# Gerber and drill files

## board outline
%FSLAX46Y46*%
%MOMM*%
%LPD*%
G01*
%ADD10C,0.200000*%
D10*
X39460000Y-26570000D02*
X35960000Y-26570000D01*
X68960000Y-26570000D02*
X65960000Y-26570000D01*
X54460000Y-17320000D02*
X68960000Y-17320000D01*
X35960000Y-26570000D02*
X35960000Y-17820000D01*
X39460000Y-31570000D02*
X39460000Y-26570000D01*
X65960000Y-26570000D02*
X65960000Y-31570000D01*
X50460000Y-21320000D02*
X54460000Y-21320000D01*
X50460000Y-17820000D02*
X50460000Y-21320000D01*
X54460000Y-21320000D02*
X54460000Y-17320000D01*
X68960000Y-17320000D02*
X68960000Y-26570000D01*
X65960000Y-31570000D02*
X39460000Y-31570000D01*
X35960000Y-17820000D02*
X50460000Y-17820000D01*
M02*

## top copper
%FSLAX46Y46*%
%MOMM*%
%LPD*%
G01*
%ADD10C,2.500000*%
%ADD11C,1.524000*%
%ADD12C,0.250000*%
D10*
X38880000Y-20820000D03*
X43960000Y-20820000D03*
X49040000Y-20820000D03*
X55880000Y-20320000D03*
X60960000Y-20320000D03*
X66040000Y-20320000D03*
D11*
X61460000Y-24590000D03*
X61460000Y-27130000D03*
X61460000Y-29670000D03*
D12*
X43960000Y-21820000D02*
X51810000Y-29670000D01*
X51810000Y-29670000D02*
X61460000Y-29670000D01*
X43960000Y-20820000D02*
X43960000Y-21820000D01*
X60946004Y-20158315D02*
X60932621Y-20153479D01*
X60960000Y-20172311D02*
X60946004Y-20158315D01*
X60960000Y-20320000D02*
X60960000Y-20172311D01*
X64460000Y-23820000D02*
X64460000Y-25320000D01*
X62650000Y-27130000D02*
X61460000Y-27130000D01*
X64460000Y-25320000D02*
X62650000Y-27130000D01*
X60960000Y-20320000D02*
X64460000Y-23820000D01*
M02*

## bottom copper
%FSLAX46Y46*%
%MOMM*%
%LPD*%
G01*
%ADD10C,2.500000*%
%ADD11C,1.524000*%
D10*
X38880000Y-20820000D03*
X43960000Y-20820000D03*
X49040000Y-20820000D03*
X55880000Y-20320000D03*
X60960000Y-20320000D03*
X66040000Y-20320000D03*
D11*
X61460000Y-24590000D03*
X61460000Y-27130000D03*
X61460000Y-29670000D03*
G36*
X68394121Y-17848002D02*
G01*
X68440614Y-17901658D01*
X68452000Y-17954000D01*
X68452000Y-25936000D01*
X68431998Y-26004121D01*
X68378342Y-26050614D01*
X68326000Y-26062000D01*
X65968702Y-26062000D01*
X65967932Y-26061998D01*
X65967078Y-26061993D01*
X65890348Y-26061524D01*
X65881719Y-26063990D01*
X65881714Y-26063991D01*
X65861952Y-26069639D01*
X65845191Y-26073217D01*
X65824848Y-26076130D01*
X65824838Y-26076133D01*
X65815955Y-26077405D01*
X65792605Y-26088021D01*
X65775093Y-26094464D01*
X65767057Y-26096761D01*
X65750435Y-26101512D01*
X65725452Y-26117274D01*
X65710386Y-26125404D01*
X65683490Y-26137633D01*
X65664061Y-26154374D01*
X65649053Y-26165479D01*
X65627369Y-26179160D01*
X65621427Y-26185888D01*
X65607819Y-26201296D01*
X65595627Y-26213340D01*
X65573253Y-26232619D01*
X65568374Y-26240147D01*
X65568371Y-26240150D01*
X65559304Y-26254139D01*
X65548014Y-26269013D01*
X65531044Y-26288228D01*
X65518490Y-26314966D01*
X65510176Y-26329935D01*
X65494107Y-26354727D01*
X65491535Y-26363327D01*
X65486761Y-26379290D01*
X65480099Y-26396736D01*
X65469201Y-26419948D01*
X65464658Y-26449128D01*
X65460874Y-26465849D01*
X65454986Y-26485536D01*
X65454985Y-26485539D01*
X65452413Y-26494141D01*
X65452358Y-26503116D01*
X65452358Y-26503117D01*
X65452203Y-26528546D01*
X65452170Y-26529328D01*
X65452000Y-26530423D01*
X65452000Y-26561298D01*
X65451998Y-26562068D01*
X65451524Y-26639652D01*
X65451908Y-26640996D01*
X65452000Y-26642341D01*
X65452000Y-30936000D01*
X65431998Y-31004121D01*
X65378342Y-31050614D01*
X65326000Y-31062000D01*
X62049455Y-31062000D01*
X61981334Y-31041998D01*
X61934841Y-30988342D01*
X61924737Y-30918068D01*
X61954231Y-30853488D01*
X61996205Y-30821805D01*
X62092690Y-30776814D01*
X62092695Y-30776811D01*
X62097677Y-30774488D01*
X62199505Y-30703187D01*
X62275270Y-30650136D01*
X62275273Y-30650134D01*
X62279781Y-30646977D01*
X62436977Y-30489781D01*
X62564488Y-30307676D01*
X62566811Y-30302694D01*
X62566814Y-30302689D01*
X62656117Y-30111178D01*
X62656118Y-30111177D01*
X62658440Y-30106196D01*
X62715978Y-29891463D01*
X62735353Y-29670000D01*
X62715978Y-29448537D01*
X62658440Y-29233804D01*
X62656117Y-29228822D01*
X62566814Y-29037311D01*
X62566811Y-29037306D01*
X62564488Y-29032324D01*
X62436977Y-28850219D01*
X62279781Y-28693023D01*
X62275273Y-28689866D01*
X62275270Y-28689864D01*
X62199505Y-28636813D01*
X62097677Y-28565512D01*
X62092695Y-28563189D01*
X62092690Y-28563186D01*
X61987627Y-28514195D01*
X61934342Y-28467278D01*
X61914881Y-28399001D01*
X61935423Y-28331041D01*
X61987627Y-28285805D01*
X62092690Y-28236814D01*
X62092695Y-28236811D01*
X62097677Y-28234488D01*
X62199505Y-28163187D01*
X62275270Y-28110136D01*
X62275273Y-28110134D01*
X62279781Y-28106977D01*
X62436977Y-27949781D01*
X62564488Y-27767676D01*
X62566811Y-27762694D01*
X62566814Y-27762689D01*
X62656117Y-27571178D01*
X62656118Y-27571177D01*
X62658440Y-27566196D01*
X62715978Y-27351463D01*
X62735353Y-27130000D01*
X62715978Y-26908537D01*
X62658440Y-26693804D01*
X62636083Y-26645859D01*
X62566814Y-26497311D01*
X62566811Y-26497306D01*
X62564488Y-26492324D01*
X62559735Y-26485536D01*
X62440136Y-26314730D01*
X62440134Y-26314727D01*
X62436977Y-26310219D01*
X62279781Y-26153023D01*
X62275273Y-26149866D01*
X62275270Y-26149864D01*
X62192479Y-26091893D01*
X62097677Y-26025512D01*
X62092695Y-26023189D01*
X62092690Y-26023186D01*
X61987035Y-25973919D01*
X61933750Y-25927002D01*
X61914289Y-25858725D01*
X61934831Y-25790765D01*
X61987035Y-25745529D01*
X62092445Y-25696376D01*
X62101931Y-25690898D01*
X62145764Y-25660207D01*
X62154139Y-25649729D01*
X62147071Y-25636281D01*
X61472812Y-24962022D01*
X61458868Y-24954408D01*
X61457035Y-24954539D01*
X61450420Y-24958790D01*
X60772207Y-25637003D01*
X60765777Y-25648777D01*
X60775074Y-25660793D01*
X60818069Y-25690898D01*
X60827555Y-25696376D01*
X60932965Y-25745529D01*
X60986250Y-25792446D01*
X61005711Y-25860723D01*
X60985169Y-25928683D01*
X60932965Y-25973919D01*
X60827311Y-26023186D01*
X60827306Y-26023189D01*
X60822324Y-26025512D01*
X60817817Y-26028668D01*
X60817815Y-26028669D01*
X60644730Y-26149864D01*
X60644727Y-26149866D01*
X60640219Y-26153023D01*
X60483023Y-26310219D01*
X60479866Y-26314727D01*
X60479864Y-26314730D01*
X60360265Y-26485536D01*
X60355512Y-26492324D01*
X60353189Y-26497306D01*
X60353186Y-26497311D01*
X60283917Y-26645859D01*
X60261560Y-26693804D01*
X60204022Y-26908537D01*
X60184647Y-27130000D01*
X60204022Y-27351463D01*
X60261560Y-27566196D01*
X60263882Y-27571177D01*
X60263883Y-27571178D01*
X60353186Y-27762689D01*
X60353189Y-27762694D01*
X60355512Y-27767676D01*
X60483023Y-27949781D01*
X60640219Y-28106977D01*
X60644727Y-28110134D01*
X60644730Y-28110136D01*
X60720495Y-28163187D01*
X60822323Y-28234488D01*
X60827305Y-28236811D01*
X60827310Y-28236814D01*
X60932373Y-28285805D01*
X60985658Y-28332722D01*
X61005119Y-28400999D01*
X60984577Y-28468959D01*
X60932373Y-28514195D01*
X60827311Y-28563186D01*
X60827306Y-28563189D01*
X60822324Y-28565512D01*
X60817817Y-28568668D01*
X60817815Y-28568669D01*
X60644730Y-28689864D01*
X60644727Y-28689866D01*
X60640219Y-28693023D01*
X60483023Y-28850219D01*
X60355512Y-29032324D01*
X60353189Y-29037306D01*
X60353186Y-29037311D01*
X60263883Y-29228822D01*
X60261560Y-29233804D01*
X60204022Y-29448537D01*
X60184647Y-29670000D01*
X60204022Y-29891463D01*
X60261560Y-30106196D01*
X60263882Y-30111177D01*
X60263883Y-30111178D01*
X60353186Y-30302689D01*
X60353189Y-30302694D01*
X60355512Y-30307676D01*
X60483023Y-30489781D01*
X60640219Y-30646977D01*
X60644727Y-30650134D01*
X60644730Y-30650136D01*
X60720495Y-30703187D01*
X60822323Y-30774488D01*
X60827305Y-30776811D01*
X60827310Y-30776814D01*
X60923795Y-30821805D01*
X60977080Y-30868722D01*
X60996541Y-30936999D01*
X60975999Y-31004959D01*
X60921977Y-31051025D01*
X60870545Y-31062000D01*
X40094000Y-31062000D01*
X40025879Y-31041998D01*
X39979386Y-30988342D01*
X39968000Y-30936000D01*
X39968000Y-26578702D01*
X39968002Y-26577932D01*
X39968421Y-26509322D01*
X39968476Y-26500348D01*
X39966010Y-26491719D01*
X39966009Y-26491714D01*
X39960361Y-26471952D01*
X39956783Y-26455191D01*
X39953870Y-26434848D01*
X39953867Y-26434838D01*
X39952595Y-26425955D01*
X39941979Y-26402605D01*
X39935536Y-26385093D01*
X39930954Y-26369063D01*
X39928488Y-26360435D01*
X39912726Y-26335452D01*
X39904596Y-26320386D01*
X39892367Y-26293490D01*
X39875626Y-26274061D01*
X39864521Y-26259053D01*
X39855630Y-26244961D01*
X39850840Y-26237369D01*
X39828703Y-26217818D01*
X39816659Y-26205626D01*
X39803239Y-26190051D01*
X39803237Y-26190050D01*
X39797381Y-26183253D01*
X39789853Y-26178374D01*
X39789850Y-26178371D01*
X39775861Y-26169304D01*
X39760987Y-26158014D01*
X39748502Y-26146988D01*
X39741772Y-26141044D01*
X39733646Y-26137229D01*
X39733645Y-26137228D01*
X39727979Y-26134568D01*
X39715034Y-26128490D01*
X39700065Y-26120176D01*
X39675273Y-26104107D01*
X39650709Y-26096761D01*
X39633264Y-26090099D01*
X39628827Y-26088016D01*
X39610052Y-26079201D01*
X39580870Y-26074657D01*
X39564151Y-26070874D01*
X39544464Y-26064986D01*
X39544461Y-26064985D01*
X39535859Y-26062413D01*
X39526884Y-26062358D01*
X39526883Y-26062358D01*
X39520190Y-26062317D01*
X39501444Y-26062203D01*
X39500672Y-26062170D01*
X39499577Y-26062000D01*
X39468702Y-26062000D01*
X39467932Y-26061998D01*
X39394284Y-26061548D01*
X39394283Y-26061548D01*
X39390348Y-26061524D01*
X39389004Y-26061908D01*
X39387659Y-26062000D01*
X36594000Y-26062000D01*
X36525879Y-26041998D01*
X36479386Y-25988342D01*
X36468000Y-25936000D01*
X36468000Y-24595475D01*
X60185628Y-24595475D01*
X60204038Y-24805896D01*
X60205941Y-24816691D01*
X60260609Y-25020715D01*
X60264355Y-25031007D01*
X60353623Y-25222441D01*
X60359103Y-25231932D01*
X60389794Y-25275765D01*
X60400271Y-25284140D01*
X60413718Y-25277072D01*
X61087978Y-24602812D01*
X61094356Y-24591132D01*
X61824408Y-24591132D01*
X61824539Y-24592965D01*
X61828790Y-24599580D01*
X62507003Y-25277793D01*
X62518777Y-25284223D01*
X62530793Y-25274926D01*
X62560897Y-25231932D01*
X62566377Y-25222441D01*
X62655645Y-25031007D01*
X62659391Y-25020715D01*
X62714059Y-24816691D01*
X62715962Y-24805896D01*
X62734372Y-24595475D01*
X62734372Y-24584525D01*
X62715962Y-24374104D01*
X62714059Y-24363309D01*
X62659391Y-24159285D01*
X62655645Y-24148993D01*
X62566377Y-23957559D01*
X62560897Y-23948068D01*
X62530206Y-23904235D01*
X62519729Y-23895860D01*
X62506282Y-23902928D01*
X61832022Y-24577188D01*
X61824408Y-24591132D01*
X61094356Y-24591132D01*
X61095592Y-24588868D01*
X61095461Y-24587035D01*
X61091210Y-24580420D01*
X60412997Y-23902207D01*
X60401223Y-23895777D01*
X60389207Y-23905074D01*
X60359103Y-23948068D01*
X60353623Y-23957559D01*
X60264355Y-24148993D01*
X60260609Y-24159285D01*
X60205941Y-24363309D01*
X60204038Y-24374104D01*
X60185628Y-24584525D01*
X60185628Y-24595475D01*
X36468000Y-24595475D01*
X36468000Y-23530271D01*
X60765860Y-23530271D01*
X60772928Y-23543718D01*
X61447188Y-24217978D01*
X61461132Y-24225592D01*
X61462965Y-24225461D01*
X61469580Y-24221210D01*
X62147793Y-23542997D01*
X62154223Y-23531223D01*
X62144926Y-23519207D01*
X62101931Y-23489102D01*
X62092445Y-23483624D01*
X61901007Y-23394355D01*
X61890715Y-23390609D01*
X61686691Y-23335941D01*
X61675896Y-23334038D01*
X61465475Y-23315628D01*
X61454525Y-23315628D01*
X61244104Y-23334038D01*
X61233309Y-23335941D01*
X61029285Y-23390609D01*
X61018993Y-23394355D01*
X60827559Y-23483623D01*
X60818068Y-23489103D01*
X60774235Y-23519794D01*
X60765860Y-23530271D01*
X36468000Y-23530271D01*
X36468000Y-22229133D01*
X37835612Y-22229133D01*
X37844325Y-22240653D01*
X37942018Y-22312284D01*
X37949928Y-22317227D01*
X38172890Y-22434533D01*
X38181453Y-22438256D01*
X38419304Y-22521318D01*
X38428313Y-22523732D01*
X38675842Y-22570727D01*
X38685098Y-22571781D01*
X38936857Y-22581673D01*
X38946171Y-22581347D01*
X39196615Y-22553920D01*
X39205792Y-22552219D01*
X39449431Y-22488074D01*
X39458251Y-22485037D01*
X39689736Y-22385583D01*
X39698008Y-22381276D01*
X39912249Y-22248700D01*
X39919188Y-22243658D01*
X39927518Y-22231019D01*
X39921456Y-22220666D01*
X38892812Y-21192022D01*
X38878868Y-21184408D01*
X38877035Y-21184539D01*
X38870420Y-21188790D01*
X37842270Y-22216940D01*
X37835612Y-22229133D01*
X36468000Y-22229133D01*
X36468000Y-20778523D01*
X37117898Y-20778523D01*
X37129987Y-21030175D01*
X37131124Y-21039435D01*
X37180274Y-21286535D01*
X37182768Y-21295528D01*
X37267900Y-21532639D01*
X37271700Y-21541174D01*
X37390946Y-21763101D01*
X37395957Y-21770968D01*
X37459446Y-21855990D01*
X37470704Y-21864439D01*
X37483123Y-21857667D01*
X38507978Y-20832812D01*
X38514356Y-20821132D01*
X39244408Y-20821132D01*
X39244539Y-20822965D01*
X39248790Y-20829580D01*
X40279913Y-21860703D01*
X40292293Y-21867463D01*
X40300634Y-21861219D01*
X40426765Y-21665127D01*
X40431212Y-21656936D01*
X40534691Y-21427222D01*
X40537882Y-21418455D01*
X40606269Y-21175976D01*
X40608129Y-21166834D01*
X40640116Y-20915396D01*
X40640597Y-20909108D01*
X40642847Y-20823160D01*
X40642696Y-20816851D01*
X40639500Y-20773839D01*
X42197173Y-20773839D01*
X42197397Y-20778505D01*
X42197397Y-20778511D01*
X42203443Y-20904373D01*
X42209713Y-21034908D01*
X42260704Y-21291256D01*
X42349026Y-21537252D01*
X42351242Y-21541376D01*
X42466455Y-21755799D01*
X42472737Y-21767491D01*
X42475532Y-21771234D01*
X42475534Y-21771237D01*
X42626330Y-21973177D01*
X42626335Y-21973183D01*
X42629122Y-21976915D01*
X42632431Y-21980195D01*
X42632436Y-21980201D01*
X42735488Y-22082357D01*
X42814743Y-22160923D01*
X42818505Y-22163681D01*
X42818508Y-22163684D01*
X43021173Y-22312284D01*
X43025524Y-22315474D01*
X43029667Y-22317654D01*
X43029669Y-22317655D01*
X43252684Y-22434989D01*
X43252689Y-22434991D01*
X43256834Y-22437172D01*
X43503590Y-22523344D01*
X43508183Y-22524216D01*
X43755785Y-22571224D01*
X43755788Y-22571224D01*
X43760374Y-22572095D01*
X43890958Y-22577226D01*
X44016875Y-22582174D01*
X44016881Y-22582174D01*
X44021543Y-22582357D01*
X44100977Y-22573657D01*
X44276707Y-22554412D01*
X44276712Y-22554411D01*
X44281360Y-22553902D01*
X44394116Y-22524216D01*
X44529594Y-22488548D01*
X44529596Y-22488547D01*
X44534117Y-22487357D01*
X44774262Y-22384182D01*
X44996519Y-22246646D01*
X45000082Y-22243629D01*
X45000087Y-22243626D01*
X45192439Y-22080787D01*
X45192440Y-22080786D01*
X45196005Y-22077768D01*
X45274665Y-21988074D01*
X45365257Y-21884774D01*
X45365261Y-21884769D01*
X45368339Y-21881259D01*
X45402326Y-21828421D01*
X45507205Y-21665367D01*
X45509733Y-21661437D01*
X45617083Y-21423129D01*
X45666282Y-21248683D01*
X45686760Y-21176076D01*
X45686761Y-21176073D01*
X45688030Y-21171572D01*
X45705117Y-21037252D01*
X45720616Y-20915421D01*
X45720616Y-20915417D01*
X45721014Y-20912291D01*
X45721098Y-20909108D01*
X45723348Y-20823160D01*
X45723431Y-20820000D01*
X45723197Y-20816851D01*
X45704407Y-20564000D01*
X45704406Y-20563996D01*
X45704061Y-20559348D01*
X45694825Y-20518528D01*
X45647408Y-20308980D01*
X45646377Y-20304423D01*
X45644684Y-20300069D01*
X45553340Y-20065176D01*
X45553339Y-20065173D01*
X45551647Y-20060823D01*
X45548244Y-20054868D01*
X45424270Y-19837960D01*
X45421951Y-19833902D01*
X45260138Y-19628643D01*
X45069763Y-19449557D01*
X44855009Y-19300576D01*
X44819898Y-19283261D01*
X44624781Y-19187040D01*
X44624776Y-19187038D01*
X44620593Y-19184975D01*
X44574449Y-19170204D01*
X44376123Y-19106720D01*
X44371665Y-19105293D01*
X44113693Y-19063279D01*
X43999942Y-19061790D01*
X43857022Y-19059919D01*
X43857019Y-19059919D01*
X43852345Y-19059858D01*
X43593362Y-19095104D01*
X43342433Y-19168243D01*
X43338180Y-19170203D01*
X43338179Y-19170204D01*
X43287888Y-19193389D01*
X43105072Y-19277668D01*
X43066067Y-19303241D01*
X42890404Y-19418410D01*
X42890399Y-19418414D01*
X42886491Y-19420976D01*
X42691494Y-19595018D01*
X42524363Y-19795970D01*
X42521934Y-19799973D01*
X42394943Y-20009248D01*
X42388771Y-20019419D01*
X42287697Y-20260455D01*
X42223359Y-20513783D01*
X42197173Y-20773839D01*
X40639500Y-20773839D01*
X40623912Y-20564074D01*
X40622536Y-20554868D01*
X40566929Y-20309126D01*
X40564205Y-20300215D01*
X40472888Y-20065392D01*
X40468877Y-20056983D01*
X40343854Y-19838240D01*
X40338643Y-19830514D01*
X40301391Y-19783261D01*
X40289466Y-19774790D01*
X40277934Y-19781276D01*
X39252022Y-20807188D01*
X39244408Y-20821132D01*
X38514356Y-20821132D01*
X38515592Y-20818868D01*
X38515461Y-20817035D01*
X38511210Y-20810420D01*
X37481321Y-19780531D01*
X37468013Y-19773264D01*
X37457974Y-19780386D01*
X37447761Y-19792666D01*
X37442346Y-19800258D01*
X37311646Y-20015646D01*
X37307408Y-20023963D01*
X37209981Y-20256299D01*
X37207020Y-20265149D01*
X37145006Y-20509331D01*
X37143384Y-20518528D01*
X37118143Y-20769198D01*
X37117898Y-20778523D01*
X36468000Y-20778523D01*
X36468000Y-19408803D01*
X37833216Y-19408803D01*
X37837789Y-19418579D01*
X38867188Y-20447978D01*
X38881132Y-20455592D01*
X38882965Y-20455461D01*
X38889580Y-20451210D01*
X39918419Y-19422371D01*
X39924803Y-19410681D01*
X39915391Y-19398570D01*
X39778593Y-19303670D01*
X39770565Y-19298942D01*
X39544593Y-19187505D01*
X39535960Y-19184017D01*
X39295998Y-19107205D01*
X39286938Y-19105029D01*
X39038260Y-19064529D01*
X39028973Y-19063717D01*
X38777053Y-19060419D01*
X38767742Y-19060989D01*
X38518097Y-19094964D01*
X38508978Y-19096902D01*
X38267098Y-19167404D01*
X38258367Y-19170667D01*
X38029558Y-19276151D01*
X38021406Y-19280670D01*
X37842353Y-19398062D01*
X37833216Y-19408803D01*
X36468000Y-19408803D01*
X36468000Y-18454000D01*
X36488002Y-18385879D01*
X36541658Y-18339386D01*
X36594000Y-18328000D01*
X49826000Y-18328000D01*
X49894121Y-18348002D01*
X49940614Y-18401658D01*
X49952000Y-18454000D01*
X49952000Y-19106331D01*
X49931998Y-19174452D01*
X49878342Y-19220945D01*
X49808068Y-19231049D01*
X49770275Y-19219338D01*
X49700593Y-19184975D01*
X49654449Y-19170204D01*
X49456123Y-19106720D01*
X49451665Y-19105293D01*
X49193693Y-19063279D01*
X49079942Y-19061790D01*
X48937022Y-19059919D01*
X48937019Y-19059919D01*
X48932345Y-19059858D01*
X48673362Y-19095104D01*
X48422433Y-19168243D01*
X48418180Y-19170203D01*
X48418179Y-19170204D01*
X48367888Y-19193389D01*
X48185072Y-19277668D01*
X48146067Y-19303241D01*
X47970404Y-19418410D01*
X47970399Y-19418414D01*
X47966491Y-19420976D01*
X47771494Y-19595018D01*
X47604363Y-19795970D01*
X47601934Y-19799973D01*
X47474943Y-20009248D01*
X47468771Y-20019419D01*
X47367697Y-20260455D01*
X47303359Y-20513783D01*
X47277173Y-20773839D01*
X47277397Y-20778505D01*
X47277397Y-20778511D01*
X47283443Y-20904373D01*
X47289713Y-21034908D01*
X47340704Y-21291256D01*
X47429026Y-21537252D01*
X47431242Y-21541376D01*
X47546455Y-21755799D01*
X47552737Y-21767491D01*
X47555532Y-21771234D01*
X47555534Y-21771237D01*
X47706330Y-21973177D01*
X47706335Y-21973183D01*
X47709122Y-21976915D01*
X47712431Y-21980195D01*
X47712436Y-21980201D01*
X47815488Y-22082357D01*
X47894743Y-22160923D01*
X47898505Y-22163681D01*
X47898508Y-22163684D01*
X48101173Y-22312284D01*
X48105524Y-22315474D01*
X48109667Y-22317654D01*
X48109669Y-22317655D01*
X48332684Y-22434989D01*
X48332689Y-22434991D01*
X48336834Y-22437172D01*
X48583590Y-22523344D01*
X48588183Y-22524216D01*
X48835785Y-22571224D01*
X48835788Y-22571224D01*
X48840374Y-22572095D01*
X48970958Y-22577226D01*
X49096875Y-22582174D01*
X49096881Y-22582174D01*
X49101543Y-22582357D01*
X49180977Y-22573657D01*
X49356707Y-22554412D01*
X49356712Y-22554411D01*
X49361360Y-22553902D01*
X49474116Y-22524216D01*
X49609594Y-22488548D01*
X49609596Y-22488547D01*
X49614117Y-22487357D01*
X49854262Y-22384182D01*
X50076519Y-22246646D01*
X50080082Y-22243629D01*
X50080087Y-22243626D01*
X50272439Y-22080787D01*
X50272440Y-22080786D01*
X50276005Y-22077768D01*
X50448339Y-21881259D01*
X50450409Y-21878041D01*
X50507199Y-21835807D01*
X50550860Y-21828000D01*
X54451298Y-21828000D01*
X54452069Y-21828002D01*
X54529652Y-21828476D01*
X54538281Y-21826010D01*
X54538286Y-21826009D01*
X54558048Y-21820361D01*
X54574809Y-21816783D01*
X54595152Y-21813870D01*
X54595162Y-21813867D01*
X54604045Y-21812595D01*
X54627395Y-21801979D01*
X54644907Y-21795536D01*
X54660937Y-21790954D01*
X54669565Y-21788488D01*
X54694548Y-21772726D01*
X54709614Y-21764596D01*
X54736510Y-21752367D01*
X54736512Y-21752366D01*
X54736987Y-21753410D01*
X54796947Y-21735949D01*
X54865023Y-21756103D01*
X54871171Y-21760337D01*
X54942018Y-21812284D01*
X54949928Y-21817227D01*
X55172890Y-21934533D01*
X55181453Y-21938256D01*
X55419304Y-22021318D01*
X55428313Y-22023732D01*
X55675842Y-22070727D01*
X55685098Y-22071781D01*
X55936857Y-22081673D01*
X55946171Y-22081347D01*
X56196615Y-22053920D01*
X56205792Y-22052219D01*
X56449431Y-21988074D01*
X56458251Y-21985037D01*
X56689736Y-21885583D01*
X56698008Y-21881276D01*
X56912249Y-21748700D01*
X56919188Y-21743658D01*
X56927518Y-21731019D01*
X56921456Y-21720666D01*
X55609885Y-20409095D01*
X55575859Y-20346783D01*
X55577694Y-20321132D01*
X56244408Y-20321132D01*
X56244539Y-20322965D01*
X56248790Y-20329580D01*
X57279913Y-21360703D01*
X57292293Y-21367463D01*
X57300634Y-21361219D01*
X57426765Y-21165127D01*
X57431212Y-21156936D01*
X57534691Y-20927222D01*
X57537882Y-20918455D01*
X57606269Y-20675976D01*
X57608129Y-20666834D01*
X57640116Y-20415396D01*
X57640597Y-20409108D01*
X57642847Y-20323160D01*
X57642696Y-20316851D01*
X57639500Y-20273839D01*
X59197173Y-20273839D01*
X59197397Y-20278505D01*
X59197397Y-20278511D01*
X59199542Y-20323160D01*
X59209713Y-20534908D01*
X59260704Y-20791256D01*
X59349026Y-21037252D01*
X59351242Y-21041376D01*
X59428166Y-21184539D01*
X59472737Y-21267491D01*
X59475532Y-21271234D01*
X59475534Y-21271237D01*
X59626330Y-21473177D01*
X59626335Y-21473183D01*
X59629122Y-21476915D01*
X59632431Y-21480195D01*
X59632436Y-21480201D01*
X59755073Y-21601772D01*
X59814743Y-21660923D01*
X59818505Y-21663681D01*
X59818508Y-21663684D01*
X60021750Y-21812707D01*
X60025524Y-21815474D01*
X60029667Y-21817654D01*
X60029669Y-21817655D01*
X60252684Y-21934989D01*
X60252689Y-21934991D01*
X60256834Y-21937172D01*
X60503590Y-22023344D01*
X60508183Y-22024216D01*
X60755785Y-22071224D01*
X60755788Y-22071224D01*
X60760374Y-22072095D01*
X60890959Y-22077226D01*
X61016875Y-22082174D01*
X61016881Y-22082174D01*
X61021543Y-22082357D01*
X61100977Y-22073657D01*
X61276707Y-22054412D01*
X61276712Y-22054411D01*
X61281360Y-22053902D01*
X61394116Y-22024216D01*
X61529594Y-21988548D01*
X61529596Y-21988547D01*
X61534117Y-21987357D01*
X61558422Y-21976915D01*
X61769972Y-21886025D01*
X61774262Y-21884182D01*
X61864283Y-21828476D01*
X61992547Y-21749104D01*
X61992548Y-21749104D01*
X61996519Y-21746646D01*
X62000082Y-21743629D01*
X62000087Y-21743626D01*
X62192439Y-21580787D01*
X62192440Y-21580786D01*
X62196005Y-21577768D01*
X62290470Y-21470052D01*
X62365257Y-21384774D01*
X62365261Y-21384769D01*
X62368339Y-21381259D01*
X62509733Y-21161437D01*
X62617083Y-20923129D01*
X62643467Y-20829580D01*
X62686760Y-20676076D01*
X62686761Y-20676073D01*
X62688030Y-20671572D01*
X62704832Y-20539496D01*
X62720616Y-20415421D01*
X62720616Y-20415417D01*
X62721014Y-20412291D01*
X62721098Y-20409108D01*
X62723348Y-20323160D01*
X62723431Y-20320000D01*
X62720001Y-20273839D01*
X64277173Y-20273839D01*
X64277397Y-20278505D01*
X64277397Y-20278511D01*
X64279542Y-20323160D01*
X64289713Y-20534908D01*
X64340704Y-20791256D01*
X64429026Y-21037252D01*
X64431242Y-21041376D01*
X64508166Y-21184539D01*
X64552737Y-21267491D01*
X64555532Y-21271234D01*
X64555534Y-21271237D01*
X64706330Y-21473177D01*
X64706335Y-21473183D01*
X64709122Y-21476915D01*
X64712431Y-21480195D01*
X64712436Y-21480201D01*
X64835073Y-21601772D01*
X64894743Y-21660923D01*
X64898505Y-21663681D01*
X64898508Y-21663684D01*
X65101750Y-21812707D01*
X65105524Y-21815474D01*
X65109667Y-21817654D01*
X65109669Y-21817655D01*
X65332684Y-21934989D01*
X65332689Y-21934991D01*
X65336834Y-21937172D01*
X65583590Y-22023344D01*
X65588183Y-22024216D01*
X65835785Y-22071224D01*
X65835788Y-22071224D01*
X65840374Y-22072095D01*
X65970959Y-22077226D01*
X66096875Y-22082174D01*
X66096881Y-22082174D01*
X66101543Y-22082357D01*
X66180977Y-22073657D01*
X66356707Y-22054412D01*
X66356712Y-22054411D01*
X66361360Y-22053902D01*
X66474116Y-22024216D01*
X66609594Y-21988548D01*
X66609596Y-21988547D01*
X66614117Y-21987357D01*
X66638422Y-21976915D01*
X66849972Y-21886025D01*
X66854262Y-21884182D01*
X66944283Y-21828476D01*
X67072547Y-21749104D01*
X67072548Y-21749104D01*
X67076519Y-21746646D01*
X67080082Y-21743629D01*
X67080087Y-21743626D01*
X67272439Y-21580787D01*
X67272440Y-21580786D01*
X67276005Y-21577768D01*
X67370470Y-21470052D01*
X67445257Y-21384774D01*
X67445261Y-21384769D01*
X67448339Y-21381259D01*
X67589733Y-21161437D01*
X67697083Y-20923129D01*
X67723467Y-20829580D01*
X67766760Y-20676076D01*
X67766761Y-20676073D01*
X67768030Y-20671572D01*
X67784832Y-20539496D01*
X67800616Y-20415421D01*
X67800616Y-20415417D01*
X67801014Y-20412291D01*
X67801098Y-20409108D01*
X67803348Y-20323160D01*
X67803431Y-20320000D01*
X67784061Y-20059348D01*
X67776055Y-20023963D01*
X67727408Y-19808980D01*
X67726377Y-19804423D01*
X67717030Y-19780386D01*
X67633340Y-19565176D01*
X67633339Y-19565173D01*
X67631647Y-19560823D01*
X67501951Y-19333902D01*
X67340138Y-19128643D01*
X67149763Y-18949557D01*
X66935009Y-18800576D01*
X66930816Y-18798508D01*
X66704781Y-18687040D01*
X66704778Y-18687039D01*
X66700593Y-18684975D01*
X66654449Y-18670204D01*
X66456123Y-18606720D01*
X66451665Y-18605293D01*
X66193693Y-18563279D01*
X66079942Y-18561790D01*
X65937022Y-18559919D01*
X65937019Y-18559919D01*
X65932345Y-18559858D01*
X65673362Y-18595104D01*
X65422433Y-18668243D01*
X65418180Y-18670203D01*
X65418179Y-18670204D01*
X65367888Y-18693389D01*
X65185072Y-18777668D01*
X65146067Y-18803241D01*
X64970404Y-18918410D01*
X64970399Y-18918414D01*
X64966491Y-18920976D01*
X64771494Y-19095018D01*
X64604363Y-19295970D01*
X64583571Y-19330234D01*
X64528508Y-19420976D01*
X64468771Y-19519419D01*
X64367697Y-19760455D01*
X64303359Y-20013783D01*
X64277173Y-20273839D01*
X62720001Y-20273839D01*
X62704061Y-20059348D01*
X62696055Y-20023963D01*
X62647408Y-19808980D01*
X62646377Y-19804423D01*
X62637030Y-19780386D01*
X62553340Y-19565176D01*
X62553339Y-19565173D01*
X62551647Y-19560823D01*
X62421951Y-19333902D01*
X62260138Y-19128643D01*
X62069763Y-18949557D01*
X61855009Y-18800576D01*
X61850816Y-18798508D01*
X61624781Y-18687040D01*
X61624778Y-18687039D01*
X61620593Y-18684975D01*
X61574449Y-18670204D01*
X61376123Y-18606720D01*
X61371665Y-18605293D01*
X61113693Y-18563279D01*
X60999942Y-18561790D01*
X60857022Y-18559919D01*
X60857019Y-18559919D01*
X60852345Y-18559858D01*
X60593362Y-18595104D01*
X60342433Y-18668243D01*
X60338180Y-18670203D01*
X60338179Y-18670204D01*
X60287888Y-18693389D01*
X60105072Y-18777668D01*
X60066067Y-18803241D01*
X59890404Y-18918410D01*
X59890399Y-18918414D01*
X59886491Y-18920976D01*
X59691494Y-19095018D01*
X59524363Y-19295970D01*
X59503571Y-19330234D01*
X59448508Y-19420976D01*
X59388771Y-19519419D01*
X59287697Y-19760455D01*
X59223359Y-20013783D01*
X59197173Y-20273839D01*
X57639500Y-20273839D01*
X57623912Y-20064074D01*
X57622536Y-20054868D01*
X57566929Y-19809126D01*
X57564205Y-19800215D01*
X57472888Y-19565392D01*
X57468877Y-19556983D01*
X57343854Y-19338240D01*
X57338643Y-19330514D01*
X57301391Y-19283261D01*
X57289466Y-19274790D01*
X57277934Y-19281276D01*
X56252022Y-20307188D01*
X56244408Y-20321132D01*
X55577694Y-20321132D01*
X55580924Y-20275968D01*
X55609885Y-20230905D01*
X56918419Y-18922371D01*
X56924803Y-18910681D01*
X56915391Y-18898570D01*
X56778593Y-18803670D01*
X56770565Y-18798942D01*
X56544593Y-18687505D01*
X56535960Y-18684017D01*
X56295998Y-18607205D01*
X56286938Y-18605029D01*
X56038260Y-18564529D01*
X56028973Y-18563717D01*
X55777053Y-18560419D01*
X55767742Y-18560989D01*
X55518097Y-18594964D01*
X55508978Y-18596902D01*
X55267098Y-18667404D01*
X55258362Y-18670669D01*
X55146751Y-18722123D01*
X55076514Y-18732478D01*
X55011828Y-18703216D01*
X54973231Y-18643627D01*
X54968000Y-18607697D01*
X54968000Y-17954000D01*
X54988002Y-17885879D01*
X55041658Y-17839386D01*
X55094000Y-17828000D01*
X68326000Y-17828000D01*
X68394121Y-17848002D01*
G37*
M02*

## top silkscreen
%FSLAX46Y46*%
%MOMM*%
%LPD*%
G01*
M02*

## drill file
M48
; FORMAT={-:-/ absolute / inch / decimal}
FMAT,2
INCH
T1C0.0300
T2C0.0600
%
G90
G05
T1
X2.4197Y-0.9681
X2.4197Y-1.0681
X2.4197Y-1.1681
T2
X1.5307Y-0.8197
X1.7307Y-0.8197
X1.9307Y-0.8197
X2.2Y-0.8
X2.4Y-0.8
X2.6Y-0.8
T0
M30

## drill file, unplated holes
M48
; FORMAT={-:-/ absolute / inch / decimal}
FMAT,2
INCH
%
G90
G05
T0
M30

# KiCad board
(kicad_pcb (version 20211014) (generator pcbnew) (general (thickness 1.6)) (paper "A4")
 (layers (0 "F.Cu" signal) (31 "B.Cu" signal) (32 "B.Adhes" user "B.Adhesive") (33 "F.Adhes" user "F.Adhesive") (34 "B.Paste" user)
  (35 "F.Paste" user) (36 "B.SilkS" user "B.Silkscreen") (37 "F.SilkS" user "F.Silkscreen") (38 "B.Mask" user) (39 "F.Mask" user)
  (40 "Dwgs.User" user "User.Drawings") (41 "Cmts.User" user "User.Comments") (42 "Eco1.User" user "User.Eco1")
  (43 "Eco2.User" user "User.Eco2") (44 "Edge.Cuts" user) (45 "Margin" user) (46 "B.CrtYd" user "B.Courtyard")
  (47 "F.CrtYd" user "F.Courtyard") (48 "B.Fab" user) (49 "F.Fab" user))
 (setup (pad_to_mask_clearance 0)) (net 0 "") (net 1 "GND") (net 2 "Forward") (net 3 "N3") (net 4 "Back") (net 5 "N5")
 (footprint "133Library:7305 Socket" (layer "F.Cu") (at 43.96 20.82)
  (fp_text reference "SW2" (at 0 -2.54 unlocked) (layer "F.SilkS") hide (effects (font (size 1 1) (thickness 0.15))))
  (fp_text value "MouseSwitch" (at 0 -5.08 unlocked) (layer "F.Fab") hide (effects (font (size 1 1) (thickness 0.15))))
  (pad "1" thru_hole circle (at -5.08 0) (size 2.5 2.5) (drill 1.524) (layers *.Cu *.Mask) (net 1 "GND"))
  (pad "2" thru_hole circle (at 0 0) (size 2.5 2.5) (drill 1.524) (layers *.Cu *.Mask) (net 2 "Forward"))
  (pad "3" thru_hole circle (at 5.08 0) (size 2.5 2.5) (drill 1.524) (layers *.Cu *.Mask) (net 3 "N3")))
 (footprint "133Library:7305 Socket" (layer "F.Cu") (at 60.96 20.32)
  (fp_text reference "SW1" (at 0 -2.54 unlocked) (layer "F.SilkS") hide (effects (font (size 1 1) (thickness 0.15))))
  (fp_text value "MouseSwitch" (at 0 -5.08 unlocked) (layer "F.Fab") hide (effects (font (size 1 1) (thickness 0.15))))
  (pad "1" thru_hole circle (at -5.08 0) (size 2.5 2.5) (drill 1.524) (layers *.Cu *.Mask) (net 1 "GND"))
  (pad "2" thru_hole circle (at 0 0) (size 2.5 2.5) (drill 1.524) (layers *.Cu *.Mask) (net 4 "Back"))
  (pad "3" thru_hole circle (at 5.08 0) (size 2.5 2.5) (drill 1.524) (layers *.Cu *.Mask) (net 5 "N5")))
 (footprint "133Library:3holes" (layer "B.Cu") (at 61.46 23.32 180)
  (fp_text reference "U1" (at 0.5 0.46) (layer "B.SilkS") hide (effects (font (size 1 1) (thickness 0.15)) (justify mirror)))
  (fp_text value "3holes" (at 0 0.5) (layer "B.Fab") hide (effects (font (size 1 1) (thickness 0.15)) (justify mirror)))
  (pad "1" thru_hole circle locked (at 0 -1.27 180) (size 1.524 1.524) (drill 0.762) (layers *.Cu *.Mask) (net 1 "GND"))
  (pad "2" thru_hole circle locked (at 0 -3.81 180) (size 1.524 1.524) (drill 0.762) (layers *.Cu *.Mask) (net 4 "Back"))
  (pad "3" thru_hole circle locked (at 0 -6.35 180) (size 1.524 1.524) (drill 0.762) (layers *.Cu *.Mask) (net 2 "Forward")))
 (gr_line (start 39.46 26.57) (end 35.96 26.57) (layer "Edge.Cuts") (width 0.2))
 (gr_line (start 68.96 26.57) (end 65.96 26.57) (layer "Edge.Cuts") (width 0.2))
 (gr_line (start 54.46 17.32) (end 68.96 17.32) (layer "Edge.Cuts") (width 0.2))
 (gr_line (start 35.96 26.57) (end 35.96 17.82) (layer "Edge.Cuts") (width 0.2))
 (gr_line (start 39.46 31.57) (end 39.46 26.57) (layer "Edge.Cuts") (width 0.2))
 (gr_line (start 65.96 26.57) (end 65.96 31.57) (layer "Edge.Cuts") (width 0.2))
 (gr_line (start 50.46 21.32) (end 54.46 21.32) (layer "Edge.Cuts") (width 0.2))
 (gr_line (start 50.46 17.82) (end 50.46 21.32) (layer "Edge.Cuts") (width 0.2))
 (gr_line (start 54.46 21.32) (end 54.46 17.32) (layer "Edge.Cuts") (width 0.2))
 (gr_line (start 68.96 17.32) (end 68.96 26.57) (layer "Edge.Cuts") (width 0.2))
 (gr_line (start 65.96 31.57) (end 39.46 31.57) (layer "Edge.Cuts") (width 0.2))
 (gr_line (start 35.96 17.82) (end 50.46 17.82) (layer "Edge.Cuts") (width 0.2))
 (segment (start 43.96 21.82) (end 51.81 29.67) (width 0.25) (layer "F.Cu") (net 2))
 (segment (start 51.81 29.67) (end 61.46 29.67) (width 0.25) (layer "F.Cu") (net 2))
 (segment (start 43.96 20.82) (end 43.96 21.82) (width 0.25) (layer "F.Cu") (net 2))
 (segment (start 60.946004 20.158315) (end 60.932621 20.153479) (width 0.25) (layer "F.Cu") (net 4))
 (segment (start 60.96 20.172311) (end 60.946004 20.158315) (width 0.25) (layer "F.Cu") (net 4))
 (segment (start 60.96 20.32) (end 60.96 20.172311) (width 0.25) (layer "F.Cu") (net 4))
 (segment (start 64.46 23.82) (end 64.46 25.32) (width 0.25) (layer "F.Cu") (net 4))
 (segment (start 62.65 27.13) (end 61.46 27.13) (width 0.25) (layer "F.Cu") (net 4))
 (segment (start 64.46 25.32) (end 62.65 27.13) (width 0.25) (layer "F.Cu") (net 4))
 (segment (start 60.96 20.32) (end 64.46 23.82) (width 0.25) (layer "F.Cu") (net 4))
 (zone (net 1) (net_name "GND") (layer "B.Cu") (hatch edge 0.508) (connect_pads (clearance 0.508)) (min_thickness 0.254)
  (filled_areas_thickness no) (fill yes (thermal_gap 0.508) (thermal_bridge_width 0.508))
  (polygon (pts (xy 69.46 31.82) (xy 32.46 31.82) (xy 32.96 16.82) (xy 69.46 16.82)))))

